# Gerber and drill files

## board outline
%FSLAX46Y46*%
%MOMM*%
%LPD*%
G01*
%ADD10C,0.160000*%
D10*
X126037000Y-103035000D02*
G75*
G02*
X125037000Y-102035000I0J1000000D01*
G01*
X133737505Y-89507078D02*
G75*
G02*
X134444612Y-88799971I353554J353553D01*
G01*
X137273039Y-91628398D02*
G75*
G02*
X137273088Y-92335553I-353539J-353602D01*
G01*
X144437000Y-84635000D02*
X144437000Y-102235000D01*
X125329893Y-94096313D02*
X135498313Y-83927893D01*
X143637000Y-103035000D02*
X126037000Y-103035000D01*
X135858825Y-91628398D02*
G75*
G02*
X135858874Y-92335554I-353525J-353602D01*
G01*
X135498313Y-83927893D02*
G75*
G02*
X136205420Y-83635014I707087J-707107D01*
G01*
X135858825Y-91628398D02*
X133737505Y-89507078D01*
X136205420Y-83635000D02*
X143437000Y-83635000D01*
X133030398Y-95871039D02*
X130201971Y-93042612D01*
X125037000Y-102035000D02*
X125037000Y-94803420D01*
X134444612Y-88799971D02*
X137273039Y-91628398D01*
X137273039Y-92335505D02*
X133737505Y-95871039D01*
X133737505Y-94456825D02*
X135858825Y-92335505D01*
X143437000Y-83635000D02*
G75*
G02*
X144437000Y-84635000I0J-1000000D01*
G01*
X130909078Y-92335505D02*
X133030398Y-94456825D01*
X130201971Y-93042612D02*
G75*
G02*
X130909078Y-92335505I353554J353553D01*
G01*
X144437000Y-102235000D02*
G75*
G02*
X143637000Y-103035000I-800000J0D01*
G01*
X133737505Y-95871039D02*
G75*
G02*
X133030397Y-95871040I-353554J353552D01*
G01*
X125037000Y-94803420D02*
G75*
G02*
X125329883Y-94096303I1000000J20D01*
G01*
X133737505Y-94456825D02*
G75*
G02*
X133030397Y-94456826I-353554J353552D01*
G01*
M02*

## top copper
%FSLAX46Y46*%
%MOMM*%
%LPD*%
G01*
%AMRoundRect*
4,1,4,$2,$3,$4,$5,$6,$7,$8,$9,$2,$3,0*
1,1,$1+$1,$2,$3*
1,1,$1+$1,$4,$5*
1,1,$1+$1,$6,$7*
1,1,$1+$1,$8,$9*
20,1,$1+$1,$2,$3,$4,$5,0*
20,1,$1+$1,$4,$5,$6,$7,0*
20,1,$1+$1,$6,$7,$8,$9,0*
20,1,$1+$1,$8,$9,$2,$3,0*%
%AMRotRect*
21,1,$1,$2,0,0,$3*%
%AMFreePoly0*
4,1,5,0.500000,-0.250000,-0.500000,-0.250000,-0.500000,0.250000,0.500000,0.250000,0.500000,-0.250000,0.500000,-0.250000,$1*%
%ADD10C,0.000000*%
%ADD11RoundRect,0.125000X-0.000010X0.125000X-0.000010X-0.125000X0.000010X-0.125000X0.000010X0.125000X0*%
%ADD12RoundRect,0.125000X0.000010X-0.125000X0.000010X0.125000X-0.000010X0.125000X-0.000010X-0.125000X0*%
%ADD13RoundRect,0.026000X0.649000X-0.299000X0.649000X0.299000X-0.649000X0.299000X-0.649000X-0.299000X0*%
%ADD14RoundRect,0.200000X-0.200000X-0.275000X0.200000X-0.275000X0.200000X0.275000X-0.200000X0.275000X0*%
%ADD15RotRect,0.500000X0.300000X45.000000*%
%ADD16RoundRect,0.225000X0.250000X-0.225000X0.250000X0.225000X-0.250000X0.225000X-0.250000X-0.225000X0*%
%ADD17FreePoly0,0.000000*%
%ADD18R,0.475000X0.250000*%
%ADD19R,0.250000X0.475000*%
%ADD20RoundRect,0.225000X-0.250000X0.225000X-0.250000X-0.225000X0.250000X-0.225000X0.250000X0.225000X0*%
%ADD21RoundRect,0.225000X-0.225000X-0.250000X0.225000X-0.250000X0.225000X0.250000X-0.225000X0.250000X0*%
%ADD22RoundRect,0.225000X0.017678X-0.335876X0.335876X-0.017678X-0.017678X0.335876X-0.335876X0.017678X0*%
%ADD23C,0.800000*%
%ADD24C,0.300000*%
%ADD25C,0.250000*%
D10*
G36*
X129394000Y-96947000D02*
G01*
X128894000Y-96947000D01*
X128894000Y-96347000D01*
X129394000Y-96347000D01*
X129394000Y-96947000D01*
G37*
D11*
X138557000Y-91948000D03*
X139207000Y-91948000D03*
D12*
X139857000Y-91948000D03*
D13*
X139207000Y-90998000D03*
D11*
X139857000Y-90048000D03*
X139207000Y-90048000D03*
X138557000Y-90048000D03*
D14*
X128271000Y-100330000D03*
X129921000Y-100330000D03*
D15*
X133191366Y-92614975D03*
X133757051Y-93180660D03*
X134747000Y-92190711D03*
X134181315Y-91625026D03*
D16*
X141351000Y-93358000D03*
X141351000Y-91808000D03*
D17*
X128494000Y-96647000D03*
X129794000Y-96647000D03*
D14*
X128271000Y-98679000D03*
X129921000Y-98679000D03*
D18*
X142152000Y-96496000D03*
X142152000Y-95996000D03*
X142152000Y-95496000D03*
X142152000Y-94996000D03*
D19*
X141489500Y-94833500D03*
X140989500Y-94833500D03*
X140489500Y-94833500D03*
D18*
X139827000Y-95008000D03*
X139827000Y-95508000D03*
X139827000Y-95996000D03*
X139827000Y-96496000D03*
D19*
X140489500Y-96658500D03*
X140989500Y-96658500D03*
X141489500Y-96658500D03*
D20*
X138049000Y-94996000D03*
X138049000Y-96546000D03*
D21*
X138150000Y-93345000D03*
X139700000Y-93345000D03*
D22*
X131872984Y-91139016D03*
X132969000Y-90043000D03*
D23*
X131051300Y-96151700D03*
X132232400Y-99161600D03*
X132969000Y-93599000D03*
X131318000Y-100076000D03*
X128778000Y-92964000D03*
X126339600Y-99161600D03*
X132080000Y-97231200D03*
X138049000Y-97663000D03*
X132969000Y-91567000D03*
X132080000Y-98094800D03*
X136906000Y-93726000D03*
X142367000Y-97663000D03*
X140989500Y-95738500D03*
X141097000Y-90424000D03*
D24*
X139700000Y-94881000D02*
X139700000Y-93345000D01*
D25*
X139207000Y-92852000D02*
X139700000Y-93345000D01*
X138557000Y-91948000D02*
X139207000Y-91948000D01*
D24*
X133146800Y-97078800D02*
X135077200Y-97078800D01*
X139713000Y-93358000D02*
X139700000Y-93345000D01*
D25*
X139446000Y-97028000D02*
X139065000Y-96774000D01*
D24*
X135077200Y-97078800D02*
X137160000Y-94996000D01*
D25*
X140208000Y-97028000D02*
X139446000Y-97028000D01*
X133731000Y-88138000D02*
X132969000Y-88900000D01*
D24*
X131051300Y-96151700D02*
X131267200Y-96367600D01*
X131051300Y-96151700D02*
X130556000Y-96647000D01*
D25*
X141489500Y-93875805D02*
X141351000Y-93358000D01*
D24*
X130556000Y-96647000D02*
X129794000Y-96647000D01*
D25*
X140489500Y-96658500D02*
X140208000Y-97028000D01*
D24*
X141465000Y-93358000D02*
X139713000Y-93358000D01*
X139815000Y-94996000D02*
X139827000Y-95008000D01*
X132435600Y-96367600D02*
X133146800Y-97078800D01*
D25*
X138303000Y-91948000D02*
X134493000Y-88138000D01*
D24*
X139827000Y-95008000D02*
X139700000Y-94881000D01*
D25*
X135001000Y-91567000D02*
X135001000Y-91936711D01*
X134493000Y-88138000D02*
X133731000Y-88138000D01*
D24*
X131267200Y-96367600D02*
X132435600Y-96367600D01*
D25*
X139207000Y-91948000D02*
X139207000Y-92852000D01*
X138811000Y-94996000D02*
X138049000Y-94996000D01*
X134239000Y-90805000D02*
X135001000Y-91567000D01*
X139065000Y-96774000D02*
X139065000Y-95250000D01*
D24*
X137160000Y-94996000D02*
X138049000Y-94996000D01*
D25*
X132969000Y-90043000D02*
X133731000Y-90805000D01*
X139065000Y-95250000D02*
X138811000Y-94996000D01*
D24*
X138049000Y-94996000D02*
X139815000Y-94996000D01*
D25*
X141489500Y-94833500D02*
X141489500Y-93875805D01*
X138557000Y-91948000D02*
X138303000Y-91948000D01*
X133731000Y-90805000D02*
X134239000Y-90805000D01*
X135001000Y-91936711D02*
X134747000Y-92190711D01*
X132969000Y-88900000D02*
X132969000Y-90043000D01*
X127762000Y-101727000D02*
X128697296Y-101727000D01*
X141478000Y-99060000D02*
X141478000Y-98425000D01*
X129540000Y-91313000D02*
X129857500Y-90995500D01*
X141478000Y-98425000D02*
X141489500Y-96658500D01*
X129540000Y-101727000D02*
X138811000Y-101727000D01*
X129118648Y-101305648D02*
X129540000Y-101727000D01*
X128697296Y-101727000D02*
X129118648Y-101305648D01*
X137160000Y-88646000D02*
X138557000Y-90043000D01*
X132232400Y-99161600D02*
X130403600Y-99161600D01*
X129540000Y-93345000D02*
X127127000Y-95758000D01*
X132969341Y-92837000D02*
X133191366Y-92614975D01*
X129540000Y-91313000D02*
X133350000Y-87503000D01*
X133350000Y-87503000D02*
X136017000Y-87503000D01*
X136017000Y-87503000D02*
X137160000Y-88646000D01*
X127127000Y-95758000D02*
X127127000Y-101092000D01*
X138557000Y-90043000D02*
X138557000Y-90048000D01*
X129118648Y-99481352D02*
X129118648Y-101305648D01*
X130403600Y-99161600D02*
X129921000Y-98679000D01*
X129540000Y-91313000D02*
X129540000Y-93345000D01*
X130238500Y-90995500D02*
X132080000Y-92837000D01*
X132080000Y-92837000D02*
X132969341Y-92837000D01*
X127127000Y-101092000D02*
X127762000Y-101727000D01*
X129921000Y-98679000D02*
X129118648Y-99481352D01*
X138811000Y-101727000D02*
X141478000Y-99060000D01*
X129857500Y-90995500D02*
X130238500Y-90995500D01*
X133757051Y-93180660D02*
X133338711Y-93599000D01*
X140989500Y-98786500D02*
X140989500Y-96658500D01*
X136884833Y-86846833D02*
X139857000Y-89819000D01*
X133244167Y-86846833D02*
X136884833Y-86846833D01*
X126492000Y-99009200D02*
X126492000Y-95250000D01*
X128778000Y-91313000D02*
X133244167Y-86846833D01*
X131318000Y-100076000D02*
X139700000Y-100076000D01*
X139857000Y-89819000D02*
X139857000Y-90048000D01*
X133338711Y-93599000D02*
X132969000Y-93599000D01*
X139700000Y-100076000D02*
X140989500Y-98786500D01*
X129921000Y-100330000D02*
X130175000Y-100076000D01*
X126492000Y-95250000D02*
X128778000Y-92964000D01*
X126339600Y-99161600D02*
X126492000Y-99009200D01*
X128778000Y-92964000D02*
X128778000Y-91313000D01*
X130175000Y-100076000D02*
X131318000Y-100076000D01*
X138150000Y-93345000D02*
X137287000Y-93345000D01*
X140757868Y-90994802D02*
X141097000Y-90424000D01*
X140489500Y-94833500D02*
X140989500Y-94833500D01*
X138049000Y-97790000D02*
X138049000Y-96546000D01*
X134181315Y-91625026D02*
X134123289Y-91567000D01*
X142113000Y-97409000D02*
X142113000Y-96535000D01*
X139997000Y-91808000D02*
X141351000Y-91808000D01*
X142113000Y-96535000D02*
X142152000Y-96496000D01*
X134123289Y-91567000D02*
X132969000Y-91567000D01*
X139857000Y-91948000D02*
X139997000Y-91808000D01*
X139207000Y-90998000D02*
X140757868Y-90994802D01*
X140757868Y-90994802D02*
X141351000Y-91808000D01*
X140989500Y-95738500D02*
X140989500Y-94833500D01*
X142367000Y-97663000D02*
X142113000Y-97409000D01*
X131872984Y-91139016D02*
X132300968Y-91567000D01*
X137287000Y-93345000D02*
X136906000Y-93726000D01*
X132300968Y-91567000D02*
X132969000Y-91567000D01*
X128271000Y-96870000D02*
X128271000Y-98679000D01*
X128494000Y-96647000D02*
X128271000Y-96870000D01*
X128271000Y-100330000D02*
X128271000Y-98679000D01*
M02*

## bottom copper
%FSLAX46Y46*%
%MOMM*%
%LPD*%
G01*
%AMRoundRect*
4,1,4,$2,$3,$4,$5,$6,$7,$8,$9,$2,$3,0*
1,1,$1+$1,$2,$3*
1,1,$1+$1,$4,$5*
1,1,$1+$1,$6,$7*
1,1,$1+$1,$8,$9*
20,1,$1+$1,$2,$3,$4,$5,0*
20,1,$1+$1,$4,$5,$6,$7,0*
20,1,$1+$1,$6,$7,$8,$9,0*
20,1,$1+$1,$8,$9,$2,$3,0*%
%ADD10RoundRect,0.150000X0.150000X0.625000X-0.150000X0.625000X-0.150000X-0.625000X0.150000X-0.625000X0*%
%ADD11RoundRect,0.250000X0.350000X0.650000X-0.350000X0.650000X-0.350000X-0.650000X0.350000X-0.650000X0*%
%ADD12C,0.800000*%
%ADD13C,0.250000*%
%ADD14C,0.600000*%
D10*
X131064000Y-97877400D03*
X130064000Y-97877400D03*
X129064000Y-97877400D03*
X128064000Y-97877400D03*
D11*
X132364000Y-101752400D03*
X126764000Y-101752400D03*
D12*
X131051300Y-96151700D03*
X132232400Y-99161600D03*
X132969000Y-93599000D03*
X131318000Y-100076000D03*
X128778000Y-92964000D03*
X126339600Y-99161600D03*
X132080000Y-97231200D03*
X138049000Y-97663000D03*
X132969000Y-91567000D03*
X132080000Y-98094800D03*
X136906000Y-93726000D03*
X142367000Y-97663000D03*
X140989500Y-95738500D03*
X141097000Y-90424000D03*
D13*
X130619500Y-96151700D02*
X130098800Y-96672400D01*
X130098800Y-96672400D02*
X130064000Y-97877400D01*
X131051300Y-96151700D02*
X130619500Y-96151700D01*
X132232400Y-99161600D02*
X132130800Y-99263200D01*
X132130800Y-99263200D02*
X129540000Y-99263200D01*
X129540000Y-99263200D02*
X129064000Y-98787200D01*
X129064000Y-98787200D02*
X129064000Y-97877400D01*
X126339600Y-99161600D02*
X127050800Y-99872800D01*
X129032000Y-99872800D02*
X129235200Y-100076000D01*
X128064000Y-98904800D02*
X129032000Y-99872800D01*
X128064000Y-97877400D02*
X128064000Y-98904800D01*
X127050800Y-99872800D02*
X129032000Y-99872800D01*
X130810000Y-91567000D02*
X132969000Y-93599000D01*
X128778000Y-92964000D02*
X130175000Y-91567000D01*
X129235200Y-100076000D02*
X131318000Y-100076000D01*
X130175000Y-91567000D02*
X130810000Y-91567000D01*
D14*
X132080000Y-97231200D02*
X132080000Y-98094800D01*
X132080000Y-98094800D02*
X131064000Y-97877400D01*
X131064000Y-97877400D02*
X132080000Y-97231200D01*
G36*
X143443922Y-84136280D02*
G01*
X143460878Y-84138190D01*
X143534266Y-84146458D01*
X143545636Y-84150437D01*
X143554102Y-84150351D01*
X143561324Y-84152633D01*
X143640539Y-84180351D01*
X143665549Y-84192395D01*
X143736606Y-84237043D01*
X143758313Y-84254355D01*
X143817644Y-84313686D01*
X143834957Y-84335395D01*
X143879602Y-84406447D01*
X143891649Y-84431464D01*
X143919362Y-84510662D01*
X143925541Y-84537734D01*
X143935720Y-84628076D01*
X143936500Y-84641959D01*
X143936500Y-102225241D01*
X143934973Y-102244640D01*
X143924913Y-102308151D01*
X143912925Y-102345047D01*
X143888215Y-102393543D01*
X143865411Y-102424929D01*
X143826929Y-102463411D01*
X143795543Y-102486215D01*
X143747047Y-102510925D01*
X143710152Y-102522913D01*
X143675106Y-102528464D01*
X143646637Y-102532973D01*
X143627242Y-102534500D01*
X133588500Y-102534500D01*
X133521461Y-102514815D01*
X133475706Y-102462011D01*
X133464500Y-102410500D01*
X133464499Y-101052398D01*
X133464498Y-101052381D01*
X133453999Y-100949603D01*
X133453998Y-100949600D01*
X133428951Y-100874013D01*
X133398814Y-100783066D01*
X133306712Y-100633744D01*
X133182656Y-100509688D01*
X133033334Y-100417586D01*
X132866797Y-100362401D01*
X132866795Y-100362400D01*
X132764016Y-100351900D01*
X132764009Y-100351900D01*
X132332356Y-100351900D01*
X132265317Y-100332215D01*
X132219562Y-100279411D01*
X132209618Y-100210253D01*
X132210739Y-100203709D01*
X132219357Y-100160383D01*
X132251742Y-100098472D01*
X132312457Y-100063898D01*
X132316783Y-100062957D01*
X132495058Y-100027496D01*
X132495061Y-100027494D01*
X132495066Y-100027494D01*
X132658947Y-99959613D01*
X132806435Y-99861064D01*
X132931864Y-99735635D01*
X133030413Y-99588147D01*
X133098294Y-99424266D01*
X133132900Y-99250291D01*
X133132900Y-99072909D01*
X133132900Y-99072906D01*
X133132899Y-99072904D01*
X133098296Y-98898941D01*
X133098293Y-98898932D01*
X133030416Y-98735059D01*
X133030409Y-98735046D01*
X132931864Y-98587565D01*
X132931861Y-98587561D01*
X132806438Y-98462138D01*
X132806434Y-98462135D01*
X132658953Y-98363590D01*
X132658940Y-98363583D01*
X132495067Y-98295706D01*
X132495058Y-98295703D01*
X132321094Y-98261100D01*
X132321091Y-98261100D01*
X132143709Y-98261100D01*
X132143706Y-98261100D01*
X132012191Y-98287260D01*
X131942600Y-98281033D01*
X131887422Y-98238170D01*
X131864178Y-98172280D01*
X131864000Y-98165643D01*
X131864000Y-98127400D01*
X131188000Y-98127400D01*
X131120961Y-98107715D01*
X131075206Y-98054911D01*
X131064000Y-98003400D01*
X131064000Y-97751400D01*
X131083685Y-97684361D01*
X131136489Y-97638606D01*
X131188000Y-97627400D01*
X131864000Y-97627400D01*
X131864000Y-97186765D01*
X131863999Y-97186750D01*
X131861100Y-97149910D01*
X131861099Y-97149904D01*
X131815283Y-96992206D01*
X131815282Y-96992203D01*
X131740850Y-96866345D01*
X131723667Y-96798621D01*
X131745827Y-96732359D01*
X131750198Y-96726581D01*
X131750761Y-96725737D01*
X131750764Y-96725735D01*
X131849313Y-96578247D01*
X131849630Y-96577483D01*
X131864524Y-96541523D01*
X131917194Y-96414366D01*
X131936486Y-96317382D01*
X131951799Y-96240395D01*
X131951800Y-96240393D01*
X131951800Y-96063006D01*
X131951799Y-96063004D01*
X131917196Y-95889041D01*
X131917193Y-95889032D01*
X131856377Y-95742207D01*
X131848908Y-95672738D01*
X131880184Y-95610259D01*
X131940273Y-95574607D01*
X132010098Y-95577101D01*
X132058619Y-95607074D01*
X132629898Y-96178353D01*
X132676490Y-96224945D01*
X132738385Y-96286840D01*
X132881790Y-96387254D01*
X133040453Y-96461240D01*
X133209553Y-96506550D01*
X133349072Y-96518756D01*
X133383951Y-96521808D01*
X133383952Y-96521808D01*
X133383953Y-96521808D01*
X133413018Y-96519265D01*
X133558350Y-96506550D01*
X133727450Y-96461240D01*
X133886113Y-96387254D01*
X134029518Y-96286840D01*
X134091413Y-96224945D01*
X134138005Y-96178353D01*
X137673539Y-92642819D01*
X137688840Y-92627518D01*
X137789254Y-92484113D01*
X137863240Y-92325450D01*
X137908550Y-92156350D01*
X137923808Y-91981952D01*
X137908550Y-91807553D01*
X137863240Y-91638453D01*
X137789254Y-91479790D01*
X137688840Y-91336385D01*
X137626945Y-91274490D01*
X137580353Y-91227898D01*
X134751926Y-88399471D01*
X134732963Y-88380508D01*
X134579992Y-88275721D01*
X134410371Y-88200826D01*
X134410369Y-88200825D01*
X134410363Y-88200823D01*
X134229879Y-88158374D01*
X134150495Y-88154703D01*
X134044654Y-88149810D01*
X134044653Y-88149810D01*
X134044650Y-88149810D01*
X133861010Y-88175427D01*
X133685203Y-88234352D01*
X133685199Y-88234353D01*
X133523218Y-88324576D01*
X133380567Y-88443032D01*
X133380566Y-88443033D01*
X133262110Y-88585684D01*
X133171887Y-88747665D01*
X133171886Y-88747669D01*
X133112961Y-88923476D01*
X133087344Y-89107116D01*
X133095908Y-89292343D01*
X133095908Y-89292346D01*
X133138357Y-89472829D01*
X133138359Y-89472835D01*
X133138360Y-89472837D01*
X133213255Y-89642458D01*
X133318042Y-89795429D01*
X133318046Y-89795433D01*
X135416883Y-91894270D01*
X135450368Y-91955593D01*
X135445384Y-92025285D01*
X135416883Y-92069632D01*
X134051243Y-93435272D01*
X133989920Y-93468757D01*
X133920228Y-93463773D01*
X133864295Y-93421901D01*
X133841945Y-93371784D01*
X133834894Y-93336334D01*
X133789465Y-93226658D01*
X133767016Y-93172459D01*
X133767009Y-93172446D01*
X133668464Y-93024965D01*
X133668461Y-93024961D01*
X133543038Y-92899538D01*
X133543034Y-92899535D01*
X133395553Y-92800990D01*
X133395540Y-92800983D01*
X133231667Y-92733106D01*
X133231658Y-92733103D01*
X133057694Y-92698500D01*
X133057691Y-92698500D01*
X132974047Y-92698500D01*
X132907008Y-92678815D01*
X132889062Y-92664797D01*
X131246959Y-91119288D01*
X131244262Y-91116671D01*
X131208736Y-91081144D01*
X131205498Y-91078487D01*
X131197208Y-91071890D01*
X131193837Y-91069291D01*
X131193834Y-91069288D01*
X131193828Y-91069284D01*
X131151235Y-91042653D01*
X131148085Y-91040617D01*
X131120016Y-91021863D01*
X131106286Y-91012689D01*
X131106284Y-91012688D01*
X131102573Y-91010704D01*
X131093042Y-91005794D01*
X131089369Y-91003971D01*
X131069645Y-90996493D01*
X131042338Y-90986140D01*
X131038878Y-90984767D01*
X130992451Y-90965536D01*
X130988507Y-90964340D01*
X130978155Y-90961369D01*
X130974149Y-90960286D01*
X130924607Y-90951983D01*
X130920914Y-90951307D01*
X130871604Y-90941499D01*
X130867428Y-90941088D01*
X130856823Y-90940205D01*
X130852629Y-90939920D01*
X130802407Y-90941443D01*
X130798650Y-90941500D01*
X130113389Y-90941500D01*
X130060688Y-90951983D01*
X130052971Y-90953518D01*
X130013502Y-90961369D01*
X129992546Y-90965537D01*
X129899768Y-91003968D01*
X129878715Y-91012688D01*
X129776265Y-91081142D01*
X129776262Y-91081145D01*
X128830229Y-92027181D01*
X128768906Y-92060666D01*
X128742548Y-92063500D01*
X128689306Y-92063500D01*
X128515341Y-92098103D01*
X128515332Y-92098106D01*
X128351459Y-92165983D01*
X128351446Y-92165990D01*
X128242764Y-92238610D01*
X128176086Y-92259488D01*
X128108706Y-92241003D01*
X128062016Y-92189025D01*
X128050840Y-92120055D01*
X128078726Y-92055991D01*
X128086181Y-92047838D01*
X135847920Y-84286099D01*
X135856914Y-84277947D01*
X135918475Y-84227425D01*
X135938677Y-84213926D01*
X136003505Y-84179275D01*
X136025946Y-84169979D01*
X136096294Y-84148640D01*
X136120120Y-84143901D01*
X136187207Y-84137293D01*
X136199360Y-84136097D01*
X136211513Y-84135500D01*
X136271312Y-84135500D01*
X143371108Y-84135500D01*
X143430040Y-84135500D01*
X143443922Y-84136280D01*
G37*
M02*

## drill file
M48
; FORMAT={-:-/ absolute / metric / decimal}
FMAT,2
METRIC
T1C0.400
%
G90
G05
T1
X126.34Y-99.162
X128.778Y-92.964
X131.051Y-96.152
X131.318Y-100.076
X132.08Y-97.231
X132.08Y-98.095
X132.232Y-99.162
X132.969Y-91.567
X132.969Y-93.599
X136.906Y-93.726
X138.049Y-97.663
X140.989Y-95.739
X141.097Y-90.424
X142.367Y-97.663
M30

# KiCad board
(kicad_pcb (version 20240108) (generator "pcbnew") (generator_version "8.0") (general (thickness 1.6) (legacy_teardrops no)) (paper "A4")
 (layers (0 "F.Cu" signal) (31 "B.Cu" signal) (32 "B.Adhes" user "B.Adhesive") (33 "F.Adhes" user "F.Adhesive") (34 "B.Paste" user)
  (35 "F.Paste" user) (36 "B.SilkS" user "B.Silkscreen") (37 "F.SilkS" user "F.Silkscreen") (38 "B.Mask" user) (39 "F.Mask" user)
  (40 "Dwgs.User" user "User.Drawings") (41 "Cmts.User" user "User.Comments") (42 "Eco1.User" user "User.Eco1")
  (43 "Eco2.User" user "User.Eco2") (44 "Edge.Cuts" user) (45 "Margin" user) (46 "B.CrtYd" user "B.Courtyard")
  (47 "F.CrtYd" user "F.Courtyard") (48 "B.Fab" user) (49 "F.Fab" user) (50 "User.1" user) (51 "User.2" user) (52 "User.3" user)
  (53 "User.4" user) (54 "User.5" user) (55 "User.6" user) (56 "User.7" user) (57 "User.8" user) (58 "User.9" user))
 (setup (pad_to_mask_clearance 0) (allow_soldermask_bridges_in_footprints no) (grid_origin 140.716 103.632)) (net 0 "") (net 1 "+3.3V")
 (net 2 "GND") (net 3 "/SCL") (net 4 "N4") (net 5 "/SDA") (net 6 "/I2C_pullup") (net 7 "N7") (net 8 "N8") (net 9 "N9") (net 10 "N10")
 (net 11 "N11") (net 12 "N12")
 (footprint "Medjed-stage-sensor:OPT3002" (layer "F.Cu") (at 139.207 90.998 90)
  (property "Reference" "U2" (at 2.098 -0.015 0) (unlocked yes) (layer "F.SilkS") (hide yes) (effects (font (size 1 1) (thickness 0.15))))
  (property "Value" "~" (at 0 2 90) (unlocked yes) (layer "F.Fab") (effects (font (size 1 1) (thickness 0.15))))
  (pad "1" smd roundrect (at -0.95 -0.65 270) (size 0.5 0.25) (layers "F.Cu" "F.Paste" "F.Mask") (roundrect_rratio 0.5) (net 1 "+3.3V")
   (thermal_bridge_angle 45))
  (pad "2" smd roundrect (at -0.95 0 270) (size 0.5 0.25) (layers "F.Cu" "F.Paste" "F.Mask") (roundrect_rratio 0.5) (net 1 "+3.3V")
   (thermal_bridge_angle 45))
  (pad "3" smd roundrect (at -0.95 0.65 90) (size 0.5 0.25) (layers "F.Cu" "F.Paste" "F.Mask") (roundrect_rratio 0.5) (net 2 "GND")
   (thermal_bridge_angle 45))
  (pad "3" smd roundrect (at 0 0 90) (size 0.65 1.35) (layers "F.Cu" "F.Paste" "F.Mask") (roundrect_rratio 0.04) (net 2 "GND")
   (thermal_bridge_angle 45))
  (pad "4" smd roundrect (at 0.95 0.65 270) (size 0.5 0.25) (layers "F.Cu" "F.Paste" "F.Mask") (roundrect_rratio 0.5) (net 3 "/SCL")
   (thermal_bridge_angle 45))
  (pad "5" smd roundrect (at 0.95 0 270) (size 0.5 0.25) (layers "F.Cu" "F.Paste" "F.Mask") (roundrect_rratio 0.5) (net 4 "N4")
   (thermal_bridge_angle 45))
  (pad "6" smd roundrect (at 0.95 -0.65 270) (size 0.5 0.25) (layers "F.Cu" "F.Paste" "F.Mask") (roundrect_rratio 0.5) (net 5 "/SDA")
   (thermal_bridge_angle 45)))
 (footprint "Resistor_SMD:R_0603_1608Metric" (layer "F.Cu") (at 129.096 100.33)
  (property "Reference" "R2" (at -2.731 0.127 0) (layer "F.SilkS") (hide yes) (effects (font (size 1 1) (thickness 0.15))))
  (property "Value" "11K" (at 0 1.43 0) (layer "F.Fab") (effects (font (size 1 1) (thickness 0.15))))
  (pad "1" smd roundrect (at -0.825 0) (size 0.8 0.95) (layers "F.Cu" "F.Paste" "F.Mask") (roundrect_rratio 0.25) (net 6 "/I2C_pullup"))
  (pad "2" smd roundrect (at 0.825 0) (size 0.8 0.95) (layers "F.Cu" "F.Paste" "F.Mask") (roundrect_rratio 0.25) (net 3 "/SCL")))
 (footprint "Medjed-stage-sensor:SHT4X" (layer "F.Cu") (at 133.969183 92.402843 45)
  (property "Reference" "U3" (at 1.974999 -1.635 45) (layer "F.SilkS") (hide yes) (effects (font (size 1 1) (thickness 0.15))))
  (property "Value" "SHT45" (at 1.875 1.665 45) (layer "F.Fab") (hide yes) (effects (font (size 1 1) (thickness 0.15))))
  (pad "1" smd rect (at -0.7 -0.4 45) (size 0.5 0.3) (layers "F.Cu" "F.Paste" "F.Mask") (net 5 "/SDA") (solder_mask_margin 0.102))
  (pad "2" smd rect (at -0.7 0.4 45) (size 0.5 0.3) (layers "F.Cu" "F.Paste" "F.Mask") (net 3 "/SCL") (solder_mask_margin 0.102))
  (pad "3" smd rect (at 0.7 0.4 45) (size 0.5 0.3) (layers "F.Cu" "F.Paste" "F.Mask") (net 1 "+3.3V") (solder_mask_margin 0.102))
  (pad "4" smd rect (at 0.7 -0.4 45) (size 0.5 0.3) (layers "F.Cu" "F.Paste" "F.Mask") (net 2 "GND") (solder_mask_margin 0.102)))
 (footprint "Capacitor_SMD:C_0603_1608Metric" (layer "F.Cu") (at 141.351 92.583 90)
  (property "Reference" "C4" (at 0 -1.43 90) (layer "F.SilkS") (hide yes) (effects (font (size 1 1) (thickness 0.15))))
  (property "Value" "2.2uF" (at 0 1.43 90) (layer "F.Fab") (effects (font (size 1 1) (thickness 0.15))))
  (pad "1" smd roundrect (at -0.775 0 90) (size 0.9 0.95) (layers "F.Cu" "F.Paste" "F.Mask") (roundrect_rratio 0.25) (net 1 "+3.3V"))
  (pad "2" smd roundrect (at 0.775 0 90) (size 0.9 0.95) (layers "F.Cu" "F.Paste" "F.Mask") (roundrect_rratio 0.25) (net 2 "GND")))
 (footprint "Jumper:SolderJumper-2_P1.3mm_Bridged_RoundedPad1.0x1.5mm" (layer "F.Cu") (at 129.144 96.647)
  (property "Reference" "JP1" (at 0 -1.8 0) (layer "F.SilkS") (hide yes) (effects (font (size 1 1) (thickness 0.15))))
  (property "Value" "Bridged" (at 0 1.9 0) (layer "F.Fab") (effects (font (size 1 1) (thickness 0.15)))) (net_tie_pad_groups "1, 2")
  (fp_poly (pts (xy 0.25 -0.3) (xy -0.25 -0.3) (xy -0.25 0.3) (xy 0.25 0.3)) (stroke (width 0) (type solid)) (fill solid) (layer "F.Cu"))
  (pad "1" smd custom (at -0.65 0) (size 1 0.5) (layers "F.Cu" "F.Mask") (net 6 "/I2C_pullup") (zone_connect 2) (thermal_bridge_angle 45)
   (options (clearance outline) (anchor rect)) (primitives))
  (pad "2" smd custom (at 0.65 0) (size 1 0.5) (layers "F.Cu" "F.Mask") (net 1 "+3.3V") (zone_connect 2) (thermal_bridge_angle 45)
   (options (clearance outline) (anchor rect)) (primitives)))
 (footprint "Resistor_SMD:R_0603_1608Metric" (layer "F.Cu") (at 129.096 98.679)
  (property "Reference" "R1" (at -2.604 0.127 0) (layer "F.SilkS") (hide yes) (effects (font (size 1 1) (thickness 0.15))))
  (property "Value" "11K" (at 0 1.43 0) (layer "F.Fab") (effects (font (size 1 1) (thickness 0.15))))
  (pad "1" smd roundrect (at -0.825 0) (size 0.8 0.95) (layers "F.Cu" "F.Paste" "F.Mask") (roundrect_rratio 0.25) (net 6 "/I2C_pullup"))
  (pad "2" smd roundrect (at 0.825 0) (size 0.8 0.95) (layers "F.Cu" "F.Paste" "F.Mask") (roundrect_rratio 0.25) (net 5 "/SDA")))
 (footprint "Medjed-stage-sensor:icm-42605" (layer "F.Cu") (at 140.9895 95.746 180)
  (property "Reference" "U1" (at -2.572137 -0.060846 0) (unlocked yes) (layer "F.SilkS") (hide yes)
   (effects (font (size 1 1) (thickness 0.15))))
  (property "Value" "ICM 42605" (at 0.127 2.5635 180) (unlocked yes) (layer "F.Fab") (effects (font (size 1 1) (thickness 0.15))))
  (pad "1" smd rect (at -1.1625 -0.75 270) (size 0.25 0.475) (layers "F.Cu" "F.Paste" "F.Mask") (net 2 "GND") (thermal_bridge_angle 45))
  (pad "2" smd rect (at -1.1625 -0.25 270) (size 0.25 0.475) (layers "F.Cu" "F.Paste" "F.Mask") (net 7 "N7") (thermal_bridge_angle 45))
  (pad "3" smd rect (at -1.1625 0.25 270) (size 0.25 0.475) (layers "F.Cu" "F.Paste" "F.Mask") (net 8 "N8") (thermal_bridge_angle 45))
  (pad "4" smd rect (at -1.1625 0.75 270) (size 0.25 0.475) (layers "F.Cu" "F.Paste" "F.Mask") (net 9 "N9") (thermal_bridge_angle 45))
  (pad "5" smd rect (at -0.5 0.9125 180) (size 0.25 0.475) (layers "F.Cu" "F.Paste" "F.Mask") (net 1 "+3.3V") (thermal_bridge_angle 45))
  (pad "6" smd rect (at 0 0.9125 180) (size 0.25 0.475) (layers "F.Cu" "F.Paste" "F.Mask") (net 2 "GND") (thermal_bridge_angle 45))
  (pad "7" smd rect (at 0.5 0.9125 180) (size 0.25 0.475) (layers "F.Cu" "F.Paste" "F.Mask") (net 2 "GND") (thermal_bridge_angle 45))
  (pad "8" smd rect (at 1.1625 0.738 270) (size 0.25 0.475) (layers "F.Cu" "F.Paste" "F.Mask") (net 1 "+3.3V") (thermal_bridge_angle 45))
  (pad "9" smd rect (at 1.1625 0.238 270) (size 0.25 0.475) (layers "F.Cu" "F.Paste" "F.Mask") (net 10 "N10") (thermal_bridge_angle 45))
  (pad "10" smd rect (at 1.1625 -0.25 270) (size 0.25 0.475) (layers "F.Cu" "F.Paste" "F.Mask") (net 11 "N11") (thermal_bridge_angle 45))
  (pad "11" smd rect (at 1.1625 -0.75 270) (size 0.25 0.475) (layers "F.Cu" "F.Paste" "F.Mask") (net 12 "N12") (thermal_bridge_angle 45))
  (pad "12" smd rect (at 0.5 -0.9125 180) (size 0.25 0.475) (layers "F.Cu" "F.Paste" "F.Mask") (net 1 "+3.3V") (thermal_bridge_angle 45))
  (pad "13" smd rect (at 0 -0.9125 180) (size 0.25 0.475) (layers "F.Cu" "F.Paste" "F.Mask") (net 3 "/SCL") (thermal_bridge_angle 45))
  (pad "14" smd rect (at -0.5 -0.9125 180) (size 0.25 0.475) (layers "F.Cu" "F.Paste" "F.Mask") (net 5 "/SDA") (thermal_bridge_angle 45)))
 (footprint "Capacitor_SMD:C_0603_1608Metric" (layer "F.Cu") (at 138.049 95.771 -90)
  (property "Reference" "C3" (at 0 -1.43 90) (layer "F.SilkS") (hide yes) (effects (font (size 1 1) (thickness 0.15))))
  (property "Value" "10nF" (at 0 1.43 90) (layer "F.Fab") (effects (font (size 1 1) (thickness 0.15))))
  (pad "1" smd roundrect (at -0.775 0 270) (size 0.9 0.95) (layers "F.Cu" "F.Paste" "F.Mask") (roundrect_rratio 0.25) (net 1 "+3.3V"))
  (pad "2" smd roundrect (at 0.775 0 270) (size 0.9 0.95) (layers "F.Cu" "F.Paste" "F.Mask") (roundrect_rratio 0.25) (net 2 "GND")))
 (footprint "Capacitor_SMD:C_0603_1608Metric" (layer "F.Cu") (at 138.925 93.345)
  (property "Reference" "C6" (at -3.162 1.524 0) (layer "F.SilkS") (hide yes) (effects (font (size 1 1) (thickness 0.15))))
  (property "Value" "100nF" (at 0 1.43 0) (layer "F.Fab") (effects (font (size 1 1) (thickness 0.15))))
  (pad "1" smd roundrect (at -0.775 0) (size 0.9 0.95) (layers "F.Cu" "F.Paste" "F.Mask") (roundrect_rratio 0.25) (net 2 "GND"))
  (pad "2" smd roundrect (at 0.775 0) (size 0.9 0.95) (layers "F.Cu" "F.Paste" "F.Mask") (roundrect_rratio 0.25) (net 1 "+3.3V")))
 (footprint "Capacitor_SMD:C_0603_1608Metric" (layer "F.Cu") (at 132.420992 90.591008 45)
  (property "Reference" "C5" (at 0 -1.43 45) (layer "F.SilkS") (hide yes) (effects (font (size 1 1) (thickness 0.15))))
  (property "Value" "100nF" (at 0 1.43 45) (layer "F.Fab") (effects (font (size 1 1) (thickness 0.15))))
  (pad "1" smd roundrect (at -0.775 0 45) (size 0.9 0.95) (layers "F.Cu" "F.Paste" "F.Mask") (roundrect_rratio 0.25) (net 2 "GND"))
  (pad "2" smd roundrect (at 0.775 0 45) (size 0.9 0.95) (layers "F.Cu" "F.Paste" "F.Mask") (roundrect_rratio 0.25) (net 1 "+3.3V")))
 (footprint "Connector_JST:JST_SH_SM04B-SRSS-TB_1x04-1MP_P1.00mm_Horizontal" (layer "B.Cu") (at 129.564 99.8774 180)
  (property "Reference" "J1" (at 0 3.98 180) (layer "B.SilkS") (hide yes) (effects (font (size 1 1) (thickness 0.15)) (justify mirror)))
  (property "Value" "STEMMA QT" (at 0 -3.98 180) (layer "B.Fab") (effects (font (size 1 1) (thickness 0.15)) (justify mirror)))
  (pad "1" smd roundrect (at -1.5 2 180) (size 0.6 1.55) (layers "B.Cu" "B.Paste" "B.Mask") (roundrect_rratio 0.25) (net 2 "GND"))
  (pad "2" smd roundrect (at -0.5 2 180) (size 0.6 1.55) (layers "B.Cu" "B.Paste" "B.Mask") (roundrect_rratio 0.25) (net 1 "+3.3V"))
  (pad "3" smd roundrect (at 0.5 2 180) (size 0.6 1.55) (layers "B.Cu" "B.Paste" "B.Mask") (roundrect_rratio 0.25) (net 5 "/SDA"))
  (pad "4" smd roundrect (at 1.5 2 180) (size 0.6 1.55) (layers "B.Cu" "B.Paste" "B.Mask") (roundrect_rratio 0.25) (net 3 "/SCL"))
  (pad "MP" smd roundrect (at -2.8 -1.875 180) (size 1.2 1.8) (layers "B.Cu" "B.Paste" "B.Mask") (roundrect_rratio 0.208333))
  (pad "MP" smd roundrect (at 2.8 -1.875 180) (size 1.2 1.8) (layers "B.Cu" "B.Paste" "B.Mask") (roundrect_rratio 0.208333)))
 (gr_arc (start 126.037 103.035) (mid 125.329893 102.742107) (end 125.037 102.035) (stroke (width 0.16) (type solid)) (layer "Edge.Cuts"))
 (gr_arc (start 133.737505 89.507078) (mid 133.737505 88.799971) (end 134.444612 88.799971) (stroke (width 0.16) (type solid))
  (layer "Edge.Cuts"))
 (gr_arc (start 137.273039 91.628398) (mid 137.419486 91.981952) (end 137.273039 92.335505) (stroke (width 0.16) (type solid))
  (layer "Edge.Cuts"))
 (gr_line (start 144.437 84.635) (end 144.437 102.235) (stroke (width 0.16) (type solid)) (layer "Edge.Cuts"))
 (gr_line (start 125.329893 94.096313) (end 135.498313 83.927893) (stroke (width 0.16) (type solid)) (layer "Edge.Cuts"))
 (gr_line (start 143.637 103.035) (end 126.037 103.035) (stroke (width 0.16) (type solid)) (layer "Edge.Cuts"))
 (gr_arc (start 135.858825 91.628398) (mid 136.005272 91.981952) (end 135.858825 92.335505) (stroke (width 0.16) (type solid))
  (layer "Edge.Cuts"))
 (gr_arc (start 135.498313 83.927893) (mid 135.822737 83.71112) (end 136.20542 83.635) (stroke (width 0.16) (type solid))
  (layer "Edge.Cuts"))
 (gr_line (start 135.858825 91.628398) (end 133.737505 89.507078) (stroke (width 0.16) (type solid)) (layer "Edge.Cuts"))
 (gr_line (start 136.20542 83.635) (end 143.437 83.635) (stroke (width 0.16) (type solid)) (layer "Edge.Cuts"))
 (gr_line (start 133.030398 95.871039) (end 130.201971 93.042612) (stroke (width 0.16) (type solid)) (layer "Edge.Cuts"))
 (gr_line (start 125.037 102.035) (end 125.037 94.80342) (stroke (width 0.16) (type solid)) (layer "Edge.Cuts"))
 (gr_line (start 134.444612 88.799971) (end 137.273039 91.628398) (stroke (width 0.16) (type solid)) (layer "Edge.Cuts"))
 (gr_line (start 137.273039 92.335505) (end 133.737505 95.871039) (stroke (width 0.16) (type solid)) (layer "Edge.Cuts"))
 (gr_line (start 133.737505 94.456825) (end 135.858825 92.335505) (stroke (width 0.16) (type solid)) (layer "Edge.Cuts"))
 (gr_arc (start 143.437 83.635) (mid 144.144107 83.927893) (end 144.437 84.635) (stroke (width 0.16) (type solid)) (layer "Edge.Cuts"))
 (gr_line (start 130.909078 92.335505) (end 133.030398 94.456825) (stroke (width 0.16) (type solid)) (layer "Edge.Cuts"))
 (gr_arc (start 130.201971 93.042612) (mid 130.201971 92.335505) (end 130.909078 92.335505) (stroke (width 0.16) (type solid))
  (layer "Edge.Cuts"))
 (gr_arc (start 144.437 102.235) (mid 144.202685 102.800685) (end 143.637 103.035) (stroke (width 0.16) (type solid)) (layer "Edge.Cuts"))
 (gr_arc (start 133.737505 95.871039) (mid 133.383952 96.017486) (end 133.030398 95.871039) (stroke (width 0.16) (type solid))
  (layer "Edge.Cuts"))
 (gr_arc (start 125.037 94.80342) (mid 125.11312 94.420737) (end 125.329893 94.096313) (stroke (width 0.16) (type solid))
  (layer "Edge.Cuts"))
 (gr_arc (start 133.737505 94.456825) (mid 133.383952 94.603272) (end 133.030398 94.456825) (stroke (width 0.16) (type solid))
  (layer "Edge.Cuts"))
 (segment (start 139.7 94.881) (end 139.7 93.345) (width 0.3) (layer "F.Cu") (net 1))
 (segment (start 139.207 92.852) (end 139.7 93.345) (width 0.25) (layer "F.Cu") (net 1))
 (segment (start 138.557 91.948) (end 139.207 91.948) (width 0.25) (layer "F.Cu") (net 1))
 (segment (start 133.1468 97.0788) (end 135.0772 97.0788) (width 0.3) (layer "F.Cu") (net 1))
 (segment (start 139.713 93.358) (end 139.7 93.345) (width 0.3) (layer "F.Cu") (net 1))
 (segment (start 139.446 97.028) (end 139.065 96.774) (width 0.25) (layer "F.Cu") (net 1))
 (segment (start 135.0772 97.0788) (end 137.16 94.996) (width 0.3) (layer "F.Cu") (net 1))
 (segment (start 140.208 97.028) (end 139.446 97.028) (width 0.25) (layer "F.Cu") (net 1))
 (segment (start 133.731 88.138) (end 132.969 88.9) (width 0.25) (layer "F.Cu") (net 1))
 (segment (start 131.0513 96.1517) (end 131.2672 96.3676) (width 0.3) (layer "F.Cu") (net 1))
 (segment (start 131.0513 96.1517) (end 130.556 96.647) (width 0.3) (layer "F.Cu") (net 1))
 (segment (start 141.4895 93.875805) (end 141.351 93.358) (width 0.25) (layer "F.Cu") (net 1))
 (segment (start 130.556 96.647) (end 129.794 96.647) (width 0.3) (layer "F.Cu") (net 1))
 (segment (start 140.4895 96.6585) (end 140.208 97.028) (width 0.25) (layer "F.Cu") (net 1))
 (segment (start 141.465 93.358) (end 139.713 93.358) (width 0.3) (layer "F.Cu") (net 1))
 (segment (start 139.815 94.996) (end 139.827 95.008) (width 0.3) (layer "F.Cu") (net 1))
 (segment (start 132.4356 96.3676) (end 133.1468 97.0788) (width 0.3) (layer "F.Cu") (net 1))
 (segment (start 138.303 91.948) (end 134.493 88.138) (width 0.25) (layer "F.Cu") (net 1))
 (segment (start 139.827 95.008) (end 139.7 94.881) (width 0.3) (layer "F.Cu") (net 1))
 (segment (start 135.001 91.567) (end 135.001 91.936711) (width 0.25) (layer "F.Cu") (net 1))
 (segment (start 134.493 88.138) (end 133.731 88.138) (width 0.25) (layer "F.Cu") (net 1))
 (segment (start 131.2672 96.3676) (end 132.4356 96.3676) (width 0.3) (layer "F.Cu") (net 1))
 (segment (start 139.207 91.948) (end 139.207 92.852) (width 0.25) (layer "F.Cu") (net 1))
 (segment (start 138.811 94.996) (end 138.049 94.996) (width 0.25) (layer "F.Cu") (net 1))
 (segment (start 134.239 90.805) (end 135.001 91.567) (width 0.25) (layer "F.Cu") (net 1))
 (segment (start 139.065 96.774) (end 139.065 95.25) (width 0.25) (layer "F.Cu") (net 1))
 (segment (start 137.16 94.996) (end 138.049 94.996) (width 0.3) (layer "F.Cu") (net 1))
 (segment (start 132.969 90.043) (end 133.731 90.805) (width 0.25) (layer "F.Cu") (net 1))
 (segment (start 139.065 95.25) (end 138.811 94.996) (width 0.25) (layer "F.Cu") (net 1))
 (segment (start 138.049 94.996) (end 139.815 94.996) (width 0.3) (layer "F.Cu") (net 1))
 (segment (start 141.4895 94.8335) (end 141.4895 93.875805) (width 0.25) (layer "F.Cu") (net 1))
 (segment (start 138.557 91.948) (end 138.303 91.948) (width 0.25) (layer "F.Cu") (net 1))
 (segment (start 133.731 90.805) (end 134.239 90.805) (width 0.25) (layer "F.Cu") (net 1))
 (segment (start 135.001 91.936711) (end 134.747 92.190711) (width 0.25) (layer "F.Cu") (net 1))
 (segment (start 132.969 88.9) (end 132.969 90.043) (width 0.25) (layer "F.Cu") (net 1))
 (via (at 131.0513 96.1517) (size 0.8) (drill 0.4) (layers "F.Cu" "B.Cu") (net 1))
 (segment (start 130.6195 96.1517) (end 130.0988 96.6724) (width 0.25) (layer "B.Cu") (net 1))
 (segment (start 130.0988 96.6724) (end 130.064 97.8774) (width 0.25) (layer "B.Cu") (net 1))
 (segment (start 131.0513 96.1517) (end 130.6195 96.1517) (width 0.25) (layer "B.Cu") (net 1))
 (segment (start 127.762 101.727) (end 128.697296 101.727) (width 0.25) (layer "F.Cu") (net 5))
 (segment (start 141.478 99.06) (end 141.478 98.425) (width 0.25) (layer "F.Cu") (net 5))
 (segment (start 129.54 91.313) (end 129.8575 90.9955) (width 0.25) (layer "F.Cu") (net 5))
 (segment (start 141.478 98.425) (end 141.4895 96.6585) (width 0.25) (layer "F.Cu") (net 5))
 (segment (start 129.54 101.727) (end 138.811 101.727) (width 0.25) (layer "F.Cu") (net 5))
 (segment (start 129.118648 101.305648) (end 129.54 101.727) (width 0.25) (layer "F.Cu") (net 5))
 (segment (start 128.697296 101.727) (end 129.118648 101.305648) (width 0.25) (layer "F.Cu") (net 5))
 (segment (start 137.16 88.646) (end 138.557 90.043) (width 0.25) (layer "F.Cu") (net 5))
 (segment (start 132.2324 99.1616) (end 130.4036 99.1616) (width 0.25) (layer "F.Cu") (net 5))
 (segment (start 129.54 93.345) (end 127.127 95.758) (width 0.25) (layer "F.Cu") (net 5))
 (segment (start 132.969341 92.837) (end 133.191366 92.614975) (width 0.25) (layer "F.Cu") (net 5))
 (segment (start 129.54 91.313) (end 133.35 87.503) (width 0.25) (layer "F.Cu") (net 5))
 (segment (start 133.35 87.503) (end 136.017 87.503) (width 0.25) (layer "F.Cu") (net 5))
 (segment (start 136.017 87.503) (end 137.16 88.646) (width 0.25) (layer "F.Cu") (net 5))
 (segment (start 127.127 95.758) (end 127.127 101.092) (width 0.25) (layer "F.Cu") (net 5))
 (segment (start 138.557 90.043) (end 138.557 90.048) (width 0.25) (layer "F.Cu") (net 5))
 (segment (start 129.118648 99.481352) (end 129.118648 101.305648) (width 0.25) (layer "F.Cu") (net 5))
 (segment (start 130.4036 99.1616) (end 129.921 98.679) (width 0.25) (layer "F.Cu") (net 5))
 (segment (start 129.54 91.313) (end 129.54 93.345) (width 0.25) (layer "F.Cu") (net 5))
 (segment (start 130.2385 90.9955) (end 132.08 92.837) (width 0.25) (layer "F.Cu") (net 5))
 (segment (start 132.08 92.837) (end 132.969341 92.837) (width 0.25) (layer "F.Cu") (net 5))
 (segment (start 127.127 101.092) (end 127.762 101.727) (width 0.25) (layer "F.Cu") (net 5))
 (segment (start 129.921 98.679) (end 129.118648 99.481352) (width 0.25) (layer "F.Cu") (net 5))
 (segment (start 138.811 101.727) (end 141.478 99.06) (width 0.25) (layer "F.Cu") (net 5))
 (segment (start 129.8575 90.9955) (end 130.2385 90.9955) (width 0.25) (layer "F.Cu") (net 5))
 (via (at 132.2324 99.1616) (size 0.8) (drill 0.4) (layers "F.Cu" "B.Cu") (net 5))
 (segment (start 132.2324 99.1616) (end 132.1308 99.2632) (width 0.25) (layer "B.Cu") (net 5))
 (segment (start 132.1308 99.2632) (end 129.54 99.2632) (width 0.25) (layer "B.Cu") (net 5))
 (segment (start 129.54 99.2632) (end 129.064 98.7872) (width 0.25) (layer "B.Cu") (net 5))
 (segment (start 129.064 98.7872) (end 129.064 97.8774) (width 0.25) (layer "B.Cu") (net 5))
 (segment (start 133.757051 93.18066) (end 133.338711 93.599) (width 0.25) (layer "F.Cu") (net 3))
 (segment (start 140.9895 98.7865) (end 140.9895 96.6585) (width 0.25) (layer "F.Cu") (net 3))
 (segment (start 136.884833 86.846833) (end 139.857 89.819) (width 0.25) (layer "F.Cu") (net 3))
 (segment (start 133.244167 86.846833) (end 136.884833 86.846833) (width 0.25) (layer "F.Cu") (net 3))
 (segment (start 126.492 99.0092) (end 126.492 95.25) (width 0.25) (layer "F.Cu") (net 3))
 (segment (start 128.778 91.313) (end 133.244167 86.846833) (width 0.25) (layer "F.Cu") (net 3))
 (segment (start 131.318 100.076) (end 139.7 100.076) (width 0.25) (layer "F.Cu") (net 3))
 (segment (start 139.857 89.819) (end 139.857 90.048) (width 0.25) (layer "F.Cu") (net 3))
 (segment (start 133.338711 93.599) (end 132.969 93.599) (width 0.25) (layer "F.Cu") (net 3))
 (segment (start 139.7 100.076) (end 140.9895 98.7865) (width 0.25) (layer "F.Cu") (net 3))
 (segment (start 129.921 100.33) (end 130.175 100.076) (width 0.25) (layer "F.Cu") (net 3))
 (segment (start 126.492 95.25) (end 128.778 92.964) (width 0.25) (layer "F.Cu") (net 3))
 (segment (start 126.3396 99.1616) (end 126.492 99.0092) (width 0.25) (layer "F.Cu") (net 3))
 (segment (start 128.778 92.964) (end 128.778 91.313) (width 0.25) (layer "F.Cu") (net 3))
 (segment (start 130.175 100.076) (end 131.318 100.076) (width 0.25) (layer "F.Cu") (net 3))
 (via (at 132.969 93.599) (size 0.8) (drill 0.4) (layers "F.Cu" "B.Cu") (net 3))
 (via (at 131.318 100.076) (size 0.8) (drill 0.4) (layers "F.Cu" "B.Cu") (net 3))
 (via (at 128.778 92.964) (size 0.8) (drill 0.4) (layers "F.Cu" "B.Cu") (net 3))
 (via (at 126.3396 99.1616) (size 0.8) (drill 0.4) (layers "F.Cu" "B.Cu") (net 3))
 (segment (start 126.3396 99.1616) (end 127.0508 99.8728) (width 0.25) (layer "B.Cu") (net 3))
 (segment (start 129.032 99.8728) (end 129.2352 100.076) (width 0.25) (layer "B.Cu") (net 3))
 (segment (start 128.064 98.9048) (end 129.032 99.8728) (width 0.25) (layer "B.Cu") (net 3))
 (segment (start 128.064 97.8774) (end 128.064 98.9048) (width 0.25) (layer "B.Cu") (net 3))
 (segment (start 127.0508 99.8728) (end 129.032 99.8728) (width 0.25) (layer "B.Cu") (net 3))
 (segment (start 130.81 91.567) (end 132.969 93.599) (width 0.25) (layer "B.Cu") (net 3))
 (segment (start 128.778 92.964) (end 130.175 91.567) (width 0.25) (layer "B.Cu") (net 3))
 (segment (start 129.2352 100.076) (end 131.318 100.076) (width 0.25) (layer "B.Cu") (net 3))
 (segment (start 130.175 91.567) (end 130.81 91.567) (width 0.25) (layer "B.Cu") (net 3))
 (segment (start 138.15 93.345) (end 137.287 93.345) (width 0.25) (layer "F.Cu") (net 2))
 (segment (start 140.757868 90.994802) (end 141.097 90.424) (width 0.25) (layer "F.Cu") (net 2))
 (segment (start 140.4895 94.8335) (end 140.9895 94.8335) (width 0.25) (layer "F.Cu") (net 2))
 (segment (start 138.049 97.79) (end 138.049 96.546) (width 0.25) (layer "F.Cu") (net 2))
 (segment (start 134.181315 91.625026) (end 134.123289 91.567) (width 0.25) (layer "F.Cu") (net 2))
 (segment (start 142.113 97.409) (end 142.113 96.535) (width 0.25) (layer "F.Cu") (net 2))
 (segment (start 139.997 91.808) (end 141.351 91.808) (width 0.25) (layer "F.Cu") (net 2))
 (segment (start 142.113 96.535) (end 142.152 96.496) (width 0.25) (layer "F.Cu") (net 2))
 (segment (start 134.123289 91.567) (end 132.969 91.567) (width 0.25) (layer "F.Cu") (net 2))
 (segment (start 139.857 91.948) (end 139.997 91.808) (width 0.25) (layer "F.Cu") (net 2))
 (segment (start 139.207 90.998) (end 140.757868 90.994802) (width 0.25) (layer "F.Cu") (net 2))
 (segment (start 140.757868 90.994802) (end 141.351 91.808) (width 0.25) (layer "F.Cu") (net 2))
 (segment (start 140.9895 95.7385) (end 140.9895 94.8335) (width 0.25) (layer "F.Cu") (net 2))
 (segment (start 142.367 97.663) (end 142.113 97.409) (width 0.25) (layer "F.Cu") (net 2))
 (segment (start 131.872984 91.139016) (end 132.300968 91.567) (width 0.25) (layer "F.Cu") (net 2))
 (segment (start 137.287 93.345) (end 136.906 93.726) (width 0.25) (layer "F.Cu") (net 2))
 (segment (start 132.300968 91.567) (end 132.969 91.567) (width 0.25) (layer "F.Cu") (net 2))
 (via (at 132.08 97.2312) (size 0.8) (drill 0.4) (layers "F.Cu" "B.Cu") (free yes) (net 2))
 (via (at 138.049 97.663) (size 0.8) (drill 0.4) (layers "F.Cu" "B.Cu") (free yes) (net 2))
 (via (at 132.969 91.567) (size 0.8) (drill 0.4) (layers "F.Cu" "B.Cu") (free yes) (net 2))
 (via (at 132.08 98.0948) (size 0.8) (drill 0.4) (layers "F.Cu" "B.Cu") (free yes) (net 2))
 (via (at 136.906 93.726) (size 0.8) (drill 0.4) (layers "F.Cu" "B.Cu") (free yes) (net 2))
 (via (at 142.367 97.663) (size 0.8) (drill 0.4) (layers "F.Cu" "B.Cu") (free yes) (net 2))
 (via (at 140.9895 95.7385) (size 0.8) (drill 0.4) (layers "F.Cu" "B.Cu") (free yes) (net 2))
 (via (at 141.097 90.424) (size 0.8) (drill 0.4) (layers "F.Cu" "B.Cu") (free yes) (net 2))
 (segment (start 132.08 97.2312) (end 132.08 98.0948) (width 0.6) (layer "B.Cu") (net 2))
 (segment (start 132.08 98.0948) (end 131.064 97.8774) (width 0.6) (layer "B.Cu") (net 2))
 (segment (start 131.064 97.8774) (end 132.08 97.2312) (width 0.6) (layer "B.Cu") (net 2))
 (segment (start 128.271 96.87) (end 128.271 98.679) (width 0.25) (layer "F.Cu") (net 6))
 (segment (start 128.494 96.647) (end 128.271 96.87) (width 0.25) (layer "F.Cu") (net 6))
 (segment (start 128.271 100.33) (end 128.271 98.679) (width 0.25) (layer "F.Cu") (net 6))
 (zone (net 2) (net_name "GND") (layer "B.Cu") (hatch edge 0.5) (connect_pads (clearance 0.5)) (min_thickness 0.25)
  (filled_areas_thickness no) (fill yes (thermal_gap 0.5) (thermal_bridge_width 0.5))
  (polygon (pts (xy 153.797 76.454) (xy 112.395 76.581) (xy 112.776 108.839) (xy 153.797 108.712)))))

